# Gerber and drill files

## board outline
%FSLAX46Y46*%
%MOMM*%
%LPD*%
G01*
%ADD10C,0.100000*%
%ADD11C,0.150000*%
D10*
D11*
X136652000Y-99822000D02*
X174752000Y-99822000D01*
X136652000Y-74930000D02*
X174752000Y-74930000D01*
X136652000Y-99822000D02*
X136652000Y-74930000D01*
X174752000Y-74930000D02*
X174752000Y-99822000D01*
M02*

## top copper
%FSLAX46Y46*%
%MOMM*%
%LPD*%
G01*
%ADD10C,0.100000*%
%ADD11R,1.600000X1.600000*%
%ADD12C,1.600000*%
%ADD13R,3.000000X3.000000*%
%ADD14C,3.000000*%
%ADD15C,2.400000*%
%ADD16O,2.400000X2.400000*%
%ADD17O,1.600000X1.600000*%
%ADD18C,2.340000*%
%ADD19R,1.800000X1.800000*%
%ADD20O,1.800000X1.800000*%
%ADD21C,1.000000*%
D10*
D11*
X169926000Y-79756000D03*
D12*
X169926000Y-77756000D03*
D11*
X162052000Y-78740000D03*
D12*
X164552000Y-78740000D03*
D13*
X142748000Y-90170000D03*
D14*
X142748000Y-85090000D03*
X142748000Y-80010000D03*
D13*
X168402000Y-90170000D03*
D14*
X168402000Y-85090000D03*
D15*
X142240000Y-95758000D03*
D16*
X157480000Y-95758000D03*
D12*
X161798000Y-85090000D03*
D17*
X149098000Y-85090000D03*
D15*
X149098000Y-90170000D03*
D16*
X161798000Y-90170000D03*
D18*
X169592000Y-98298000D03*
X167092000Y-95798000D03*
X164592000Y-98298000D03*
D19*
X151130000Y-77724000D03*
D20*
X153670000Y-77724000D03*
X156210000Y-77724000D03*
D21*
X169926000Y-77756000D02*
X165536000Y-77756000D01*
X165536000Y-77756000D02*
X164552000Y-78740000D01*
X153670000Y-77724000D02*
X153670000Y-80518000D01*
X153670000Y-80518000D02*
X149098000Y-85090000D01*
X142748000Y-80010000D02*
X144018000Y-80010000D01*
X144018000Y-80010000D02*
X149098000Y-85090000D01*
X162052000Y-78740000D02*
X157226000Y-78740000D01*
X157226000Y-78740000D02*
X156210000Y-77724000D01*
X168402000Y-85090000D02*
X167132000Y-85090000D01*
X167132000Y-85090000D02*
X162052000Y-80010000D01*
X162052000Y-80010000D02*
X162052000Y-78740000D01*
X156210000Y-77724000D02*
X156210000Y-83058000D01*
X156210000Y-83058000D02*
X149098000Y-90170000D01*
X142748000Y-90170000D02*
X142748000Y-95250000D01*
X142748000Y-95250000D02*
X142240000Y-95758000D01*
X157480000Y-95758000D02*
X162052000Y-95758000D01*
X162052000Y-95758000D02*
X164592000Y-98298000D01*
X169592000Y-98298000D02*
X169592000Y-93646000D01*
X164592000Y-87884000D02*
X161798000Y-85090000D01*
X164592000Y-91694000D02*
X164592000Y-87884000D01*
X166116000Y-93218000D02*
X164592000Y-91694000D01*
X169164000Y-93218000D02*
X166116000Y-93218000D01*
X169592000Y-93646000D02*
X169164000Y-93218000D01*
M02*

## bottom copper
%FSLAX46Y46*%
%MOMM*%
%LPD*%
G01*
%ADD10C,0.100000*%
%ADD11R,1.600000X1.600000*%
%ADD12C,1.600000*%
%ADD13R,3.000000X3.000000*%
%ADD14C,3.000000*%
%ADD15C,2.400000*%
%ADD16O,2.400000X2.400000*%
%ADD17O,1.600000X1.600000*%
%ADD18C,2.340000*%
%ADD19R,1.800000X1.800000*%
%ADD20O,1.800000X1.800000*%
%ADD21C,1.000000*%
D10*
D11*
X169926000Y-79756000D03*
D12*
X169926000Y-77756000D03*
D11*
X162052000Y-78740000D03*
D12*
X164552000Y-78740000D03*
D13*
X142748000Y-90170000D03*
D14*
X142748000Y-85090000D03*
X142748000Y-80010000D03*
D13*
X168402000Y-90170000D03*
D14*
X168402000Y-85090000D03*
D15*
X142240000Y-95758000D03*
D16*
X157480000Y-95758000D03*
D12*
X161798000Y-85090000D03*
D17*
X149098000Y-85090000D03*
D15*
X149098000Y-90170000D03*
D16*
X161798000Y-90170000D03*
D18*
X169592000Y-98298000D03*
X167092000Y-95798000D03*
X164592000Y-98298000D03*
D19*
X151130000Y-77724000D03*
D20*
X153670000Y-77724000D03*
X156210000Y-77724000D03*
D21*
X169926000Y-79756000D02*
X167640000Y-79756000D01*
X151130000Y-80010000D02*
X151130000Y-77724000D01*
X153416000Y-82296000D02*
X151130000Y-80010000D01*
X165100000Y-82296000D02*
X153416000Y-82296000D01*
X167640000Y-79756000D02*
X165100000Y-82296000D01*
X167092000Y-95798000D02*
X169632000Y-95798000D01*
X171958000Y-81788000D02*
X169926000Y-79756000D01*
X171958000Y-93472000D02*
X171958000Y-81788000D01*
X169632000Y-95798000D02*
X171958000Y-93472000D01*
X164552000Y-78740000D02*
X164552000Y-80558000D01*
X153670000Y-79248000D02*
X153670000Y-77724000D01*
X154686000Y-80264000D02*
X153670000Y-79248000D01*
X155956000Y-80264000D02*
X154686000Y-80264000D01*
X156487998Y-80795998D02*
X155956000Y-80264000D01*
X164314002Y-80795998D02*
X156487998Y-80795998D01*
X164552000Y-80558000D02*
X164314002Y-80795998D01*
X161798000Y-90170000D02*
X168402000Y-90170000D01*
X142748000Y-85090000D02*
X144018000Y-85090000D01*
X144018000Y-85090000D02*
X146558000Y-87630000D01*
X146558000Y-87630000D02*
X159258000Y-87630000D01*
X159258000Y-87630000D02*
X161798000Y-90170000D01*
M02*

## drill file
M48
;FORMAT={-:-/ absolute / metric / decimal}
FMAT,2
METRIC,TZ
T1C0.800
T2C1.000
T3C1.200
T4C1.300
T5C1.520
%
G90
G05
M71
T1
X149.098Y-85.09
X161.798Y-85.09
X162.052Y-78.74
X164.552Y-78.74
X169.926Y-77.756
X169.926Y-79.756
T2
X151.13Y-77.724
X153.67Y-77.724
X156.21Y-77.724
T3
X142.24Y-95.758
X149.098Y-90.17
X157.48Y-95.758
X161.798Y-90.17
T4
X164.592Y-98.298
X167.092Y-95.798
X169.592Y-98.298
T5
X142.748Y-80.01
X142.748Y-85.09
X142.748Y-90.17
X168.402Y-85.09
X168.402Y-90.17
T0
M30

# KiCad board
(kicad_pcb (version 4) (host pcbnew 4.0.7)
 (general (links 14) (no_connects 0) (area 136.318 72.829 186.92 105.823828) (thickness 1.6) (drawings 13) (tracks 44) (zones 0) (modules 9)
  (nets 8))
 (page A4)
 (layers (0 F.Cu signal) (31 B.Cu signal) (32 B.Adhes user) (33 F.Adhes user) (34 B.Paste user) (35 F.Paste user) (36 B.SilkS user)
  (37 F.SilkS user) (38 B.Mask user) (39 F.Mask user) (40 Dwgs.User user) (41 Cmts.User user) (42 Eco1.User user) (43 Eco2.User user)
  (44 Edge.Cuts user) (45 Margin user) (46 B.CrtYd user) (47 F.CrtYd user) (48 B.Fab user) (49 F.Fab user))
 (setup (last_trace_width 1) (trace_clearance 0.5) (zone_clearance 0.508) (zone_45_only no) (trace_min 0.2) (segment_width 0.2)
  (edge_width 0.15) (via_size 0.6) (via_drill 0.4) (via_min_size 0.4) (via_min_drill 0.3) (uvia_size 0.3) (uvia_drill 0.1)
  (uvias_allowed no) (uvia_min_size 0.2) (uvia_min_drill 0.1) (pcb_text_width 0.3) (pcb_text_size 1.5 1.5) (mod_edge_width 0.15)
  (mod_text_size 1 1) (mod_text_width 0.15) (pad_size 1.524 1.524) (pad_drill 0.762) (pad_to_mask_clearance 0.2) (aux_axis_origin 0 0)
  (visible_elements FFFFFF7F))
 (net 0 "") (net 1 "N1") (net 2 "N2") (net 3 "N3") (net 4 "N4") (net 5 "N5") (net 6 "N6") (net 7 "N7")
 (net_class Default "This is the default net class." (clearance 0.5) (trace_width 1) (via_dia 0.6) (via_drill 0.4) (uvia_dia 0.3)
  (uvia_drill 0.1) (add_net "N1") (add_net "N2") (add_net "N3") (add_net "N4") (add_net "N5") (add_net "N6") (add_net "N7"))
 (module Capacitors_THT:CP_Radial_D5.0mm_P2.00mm (layer F.Cu) (at 169.926 79.756 90)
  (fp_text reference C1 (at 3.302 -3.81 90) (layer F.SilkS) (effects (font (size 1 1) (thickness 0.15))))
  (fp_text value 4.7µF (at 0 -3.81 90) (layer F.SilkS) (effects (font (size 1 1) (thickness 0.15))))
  (pad 1 thru_hole rect (at 0 0 90) (size 1.6 1.6) (drill 0.8) (layers *.Cu *.Mask) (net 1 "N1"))
  (pad 2 thru_hole circle (at 2 0 90) (size 1.6 1.6) (drill 0.8) (layers *.Cu *.Mask) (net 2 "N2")))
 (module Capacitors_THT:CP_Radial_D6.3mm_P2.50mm (layer F.Cu) (at 162.052 78.74)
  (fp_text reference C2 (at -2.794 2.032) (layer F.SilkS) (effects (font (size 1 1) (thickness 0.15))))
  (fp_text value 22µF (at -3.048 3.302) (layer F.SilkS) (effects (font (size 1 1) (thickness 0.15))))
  (pad 1 thru_hole rect (at 0 0) (size 1.6 1.6) (drill 0.8) (layers *.Cu *.Mask) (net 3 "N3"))
  (pad 2 thru_hole circle (at 2.5 0) (size 1.6 1.6) (drill 0.8) (layers *.Cu *.Mask) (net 2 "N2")))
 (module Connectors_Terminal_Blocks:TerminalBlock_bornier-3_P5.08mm (layer F.Cu) (at 142.748 90.17 90)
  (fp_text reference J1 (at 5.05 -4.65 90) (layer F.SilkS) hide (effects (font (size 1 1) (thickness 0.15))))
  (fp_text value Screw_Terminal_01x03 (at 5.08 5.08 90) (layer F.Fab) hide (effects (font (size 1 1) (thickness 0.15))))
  (pad 1 thru_hole rect (at 0 0 90) (size 3 3) (drill 1.52) (layers *.Cu *.Mask) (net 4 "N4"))
  (pad 2 thru_hole circle (at 5.08 0 90) (size 3 3) (drill 1.52) (layers *.Cu *.Mask) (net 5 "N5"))
  (pad 3 thru_hole circle (at 10.16 0 90) (size 3 3) (drill 1.52) (layers *.Cu *.Mask) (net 2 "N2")))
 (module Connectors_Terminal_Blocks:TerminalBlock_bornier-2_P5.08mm (layer F.Cu) (at 168.402 90.17 90)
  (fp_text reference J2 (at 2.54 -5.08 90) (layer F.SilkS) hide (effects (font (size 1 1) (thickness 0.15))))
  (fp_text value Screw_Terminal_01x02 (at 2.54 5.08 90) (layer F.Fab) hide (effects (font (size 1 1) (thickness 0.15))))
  (pad 1 thru_hole rect (at 0 0 90) (size 3 3) (drill 1.52) (layers *.Cu *.Mask) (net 5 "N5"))
  (pad 2 thru_hole circle (at 5.08 0 90) (size 3 3) (drill 1.52) (layers *.Cu *.Mask) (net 3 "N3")))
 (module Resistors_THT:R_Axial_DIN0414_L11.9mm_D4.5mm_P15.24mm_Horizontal (layer F.Cu) (at 142.24 95.758)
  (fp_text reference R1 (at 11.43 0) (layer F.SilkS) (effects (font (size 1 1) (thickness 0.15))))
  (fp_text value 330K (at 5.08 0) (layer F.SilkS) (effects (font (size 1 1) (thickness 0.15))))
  (pad 1 thru_hole circle (at 0 0) (size 2.4 2.4) (drill 1.2) (layers *.Cu *.Mask) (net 4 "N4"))
  (pad 2 thru_hole oval (at 15.24 0) (size 2.4 2.4) (drill 1.2) (layers *.Cu *.Mask) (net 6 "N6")))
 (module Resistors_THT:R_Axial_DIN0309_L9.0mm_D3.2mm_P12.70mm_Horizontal (layer F.Cu) (at 161.798 85.09 180)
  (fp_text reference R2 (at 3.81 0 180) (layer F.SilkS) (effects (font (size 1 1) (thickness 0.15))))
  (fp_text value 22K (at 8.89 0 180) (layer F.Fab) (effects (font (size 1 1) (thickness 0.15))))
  (pad 1 thru_hole circle (at 0 0 180) (size 1.6 1.6) (drill 0.8) (layers *.Cu *.Mask) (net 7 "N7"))
  (pad 2 thru_hole oval (at 12.7 0 180) (size 1.6 1.6) (drill 0.8) (layers *.Cu *.Mask) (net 2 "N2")))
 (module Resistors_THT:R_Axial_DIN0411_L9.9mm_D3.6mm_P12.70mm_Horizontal (layer F.Cu) (at 149.098 90.17)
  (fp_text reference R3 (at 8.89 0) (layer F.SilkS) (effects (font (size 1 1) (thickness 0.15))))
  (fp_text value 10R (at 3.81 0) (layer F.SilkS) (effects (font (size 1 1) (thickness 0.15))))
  (pad 1 thru_hole circle (at 0 0) (size 2.4 2.4) (drill 1.2) (layers *.Cu *.Mask) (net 3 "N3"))
  (pad 2 thru_hole oval (at 12.7 0) (size 2.4 2.4) (drill 1.2) (layers *.Cu *.Mask) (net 5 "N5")))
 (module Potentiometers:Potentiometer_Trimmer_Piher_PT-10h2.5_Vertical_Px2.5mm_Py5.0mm (layer F.Cu) (at 164.592 98.298 90)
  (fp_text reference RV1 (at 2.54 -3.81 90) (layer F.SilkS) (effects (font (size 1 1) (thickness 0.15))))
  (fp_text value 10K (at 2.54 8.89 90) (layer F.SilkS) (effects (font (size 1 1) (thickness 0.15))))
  (pad 3 thru_hole circle (at 0 5 90) (size 2.34 2.34) (drill 1.3) (layers *.Cu *.Mask) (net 7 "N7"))
  (pad 2 thru_hole circle (at 2.5 2.5 90) (size 2.34 2.34) (drill 1.3) (layers *.Cu *.Mask) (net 1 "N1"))
  (pad 1 thru_hole circle (at 0 0 90) (size 2.34 2.34) (drill 1.3) (layers *.Cu *.Mask) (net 6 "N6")))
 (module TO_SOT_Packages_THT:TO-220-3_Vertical (layer F.Cu) (at 151.13 77.724)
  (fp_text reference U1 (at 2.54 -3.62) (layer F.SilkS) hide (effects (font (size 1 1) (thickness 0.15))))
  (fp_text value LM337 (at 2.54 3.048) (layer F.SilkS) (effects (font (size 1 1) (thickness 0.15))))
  (pad 1 thru_hole rect (at 0 0) (size 1.8 1.8) (drill 1) (layers *.Cu *.Mask) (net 1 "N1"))
  (pad 2 thru_hole oval (at 2.54 0) (size 1.8 1.8) (drill 1) (layers *.Cu *.Mask) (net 2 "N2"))
  (pad 3 thru_hole oval (at 5.08 0) (size 1.8 1.8) (drill 1) (layers *.Cu *.Mask) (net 3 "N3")))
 (gr_line (start 136.652 99.822) (end 174.752 99.822) (angle 90) (layer Edge.Cuts) (width 0.15))
 (gr_line (start 136.652 74.93) (end 174.752 74.93) (angle 90) (layer Edge.Cuts) (width 0.15))
 (gr_line (start 136.652 99.822) (end 136.652 74.93) (angle 90) (layer Edge.Cuts) (width 0.15))
 (gr_line (start 174.752 74.93) (end 174.752 99.822) (angle 90) (layer Edge.Cuts) (width 0.15))
 (segment (start 169.926 79.756) (end 167.64 79.756) (width 1) (layer B.Cu) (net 1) (status 400000))
 (segment (start 151.13 80.01) (end 151.13 77.724) (width 1) (layer B.Cu) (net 1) (status 800000))
 (segment (start 153.416 82.296) (end 151.13 80.01) (width 1) (layer B.Cu) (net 1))
 (segment (start 165.1 82.296) (end 153.416 82.296) (width 1) (layer B.Cu) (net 1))
 (segment (start 167.64 79.756) (end 165.1 82.296) (width 1) (layer B.Cu) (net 1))
 (segment (start 167.092 95.798) (end 169.632 95.798) (width 1) (layer B.Cu) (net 1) (status 400000))
 (segment (start 171.958 81.788) (end 169.926 79.756) (width 1) (layer B.Cu) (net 1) (status 800000))
 (segment (start 171.958 93.472) (end 171.958 81.788) (width 1) (layer B.Cu) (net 1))
 (segment (start 169.632 95.798) (end 171.958 93.472) (width 1) (layer B.Cu) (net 1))
 (segment (start 169.926 77.756) (end 165.536 77.756) (width 1) (layer F.Cu) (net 2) (status 400000))
 (segment (start 165.536 77.756) (end 164.552 78.74) (width 1) (layer F.Cu) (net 2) (status 800000))
 (segment (start 164.552 78.74) (end 164.552 80.558) (width 1) (layer B.Cu) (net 2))
 (segment (start 153.67 79.248) (end 153.67 77.724) (width 1) (layer B.Cu) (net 2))
 (segment (start 154.686 80.264) (end 153.67 79.248) (width 1) (layer B.Cu) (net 2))
 (segment (start 155.956 80.264) (end 154.686 80.264) (width 1) (layer B.Cu) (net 2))
 (segment (start 156.487998 80.795998) (end 155.956 80.264) (width 1) (layer B.Cu) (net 2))
 (segment (start 164.314002 80.795998) (end 156.487998 80.795998) (width 1) (layer B.Cu) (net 2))
 (segment (start 164.552 80.558) (end 164.314002 80.795998) (width 1) (layer B.Cu) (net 2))
 (segment (start 153.67 77.724) (end 153.67 80.518) (width 1) (layer F.Cu) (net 2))
 (segment (start 153.67 80.518) (end 149.098 85.09) (width 1) (layer F.Cu) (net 2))
 (segment (start 142.748 80.01) (end 144.018 80.01) (width 1) (layer F.Cu) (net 2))
 (segment (start 144.018 80.01) (end 149.098 85.09) (width 1) (layer F.Cu) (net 2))
 (segment (start 162.052 78.74) (end 157.226 78.74) (width 1) (layer F.Cu) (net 3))
 (segment (start 157.226 78.74) (end 156.21 77.724) (width 1) (layer F.Cu) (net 3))
 (segment (start 168.402 85.09) (end 167.132 85.09) (width 1) (layer F.Cu) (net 3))
 (segment (start 167.132 85.09) (end 162.052 80.01) (width 1) (layer F.Cu) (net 3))
 (segment (start 162.052 80.01) (end 162.052 78.74) (width 1) (layer F.Cu) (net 3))
 (segment (start 156.21 77.724) (end 156.21 83.058) (width 1) (layer F.Cu) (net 3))
 (segment (start 156.21 83.058) (end 149.098 90.17) (width 1) (layer F.Cu) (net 3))
 (segment (start 142.748 90.17) (end 142.748 95.25) (width 1) (layer F.Cu) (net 4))
 (segment (start 142.748 95.25) (end 142.24 95.758) (width 1) (layer F.Cu) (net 4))
 (segment (start 161.798 90.17) (end 168.402 90.17) (width 1) (layer B.Cu) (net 5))
 (segment (start 142.748 85.09) (end 144.018 85.09) (width 1) (layer B.Cu) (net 5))
 (segment (start 144.018 85.09) (end 146.558 87.63) (width 1) (layer B.Cu) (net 5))
 (segment (start 146.558 87.63) (end 159.258 87.63) (width 1) (layer B.Cu) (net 5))
 (segment (start 159.258 87.63) (end 161.798 90.17) (width 1) (layer B.Cu) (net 5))
 (segment (start 157.48 95.758) (end 162.052 95.758) (width 1) (layer F.Cu) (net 6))
 (segment (start 162.052 95.758) (end 164.592 98.298) (width 1) (layer F.Cu) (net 6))
 (segment (start 169.592 98.298) (end 169.592 93.646) (width 1) (layer F.Cu) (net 7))
 (segment (start 164.592 87.884) (end 161.798 85.09) (width 1) (layer F.Cu) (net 7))
 (segment (start 164.592 91.694) (end 164.592 87.884) (width 1) (layer F.Cu) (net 7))
 (segment (start 166.116 93.218) (end 164.592 91.694) (width 1) (layer F.Cu) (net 7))
 (segment (start 169.164 93.218) (end 166.116 93.218) (width 1) (layer F.Cu) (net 7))
 (segment (start 169.592 93.646) (end 169.164 93.218) (width 1) (layer F.Cu) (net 7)))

